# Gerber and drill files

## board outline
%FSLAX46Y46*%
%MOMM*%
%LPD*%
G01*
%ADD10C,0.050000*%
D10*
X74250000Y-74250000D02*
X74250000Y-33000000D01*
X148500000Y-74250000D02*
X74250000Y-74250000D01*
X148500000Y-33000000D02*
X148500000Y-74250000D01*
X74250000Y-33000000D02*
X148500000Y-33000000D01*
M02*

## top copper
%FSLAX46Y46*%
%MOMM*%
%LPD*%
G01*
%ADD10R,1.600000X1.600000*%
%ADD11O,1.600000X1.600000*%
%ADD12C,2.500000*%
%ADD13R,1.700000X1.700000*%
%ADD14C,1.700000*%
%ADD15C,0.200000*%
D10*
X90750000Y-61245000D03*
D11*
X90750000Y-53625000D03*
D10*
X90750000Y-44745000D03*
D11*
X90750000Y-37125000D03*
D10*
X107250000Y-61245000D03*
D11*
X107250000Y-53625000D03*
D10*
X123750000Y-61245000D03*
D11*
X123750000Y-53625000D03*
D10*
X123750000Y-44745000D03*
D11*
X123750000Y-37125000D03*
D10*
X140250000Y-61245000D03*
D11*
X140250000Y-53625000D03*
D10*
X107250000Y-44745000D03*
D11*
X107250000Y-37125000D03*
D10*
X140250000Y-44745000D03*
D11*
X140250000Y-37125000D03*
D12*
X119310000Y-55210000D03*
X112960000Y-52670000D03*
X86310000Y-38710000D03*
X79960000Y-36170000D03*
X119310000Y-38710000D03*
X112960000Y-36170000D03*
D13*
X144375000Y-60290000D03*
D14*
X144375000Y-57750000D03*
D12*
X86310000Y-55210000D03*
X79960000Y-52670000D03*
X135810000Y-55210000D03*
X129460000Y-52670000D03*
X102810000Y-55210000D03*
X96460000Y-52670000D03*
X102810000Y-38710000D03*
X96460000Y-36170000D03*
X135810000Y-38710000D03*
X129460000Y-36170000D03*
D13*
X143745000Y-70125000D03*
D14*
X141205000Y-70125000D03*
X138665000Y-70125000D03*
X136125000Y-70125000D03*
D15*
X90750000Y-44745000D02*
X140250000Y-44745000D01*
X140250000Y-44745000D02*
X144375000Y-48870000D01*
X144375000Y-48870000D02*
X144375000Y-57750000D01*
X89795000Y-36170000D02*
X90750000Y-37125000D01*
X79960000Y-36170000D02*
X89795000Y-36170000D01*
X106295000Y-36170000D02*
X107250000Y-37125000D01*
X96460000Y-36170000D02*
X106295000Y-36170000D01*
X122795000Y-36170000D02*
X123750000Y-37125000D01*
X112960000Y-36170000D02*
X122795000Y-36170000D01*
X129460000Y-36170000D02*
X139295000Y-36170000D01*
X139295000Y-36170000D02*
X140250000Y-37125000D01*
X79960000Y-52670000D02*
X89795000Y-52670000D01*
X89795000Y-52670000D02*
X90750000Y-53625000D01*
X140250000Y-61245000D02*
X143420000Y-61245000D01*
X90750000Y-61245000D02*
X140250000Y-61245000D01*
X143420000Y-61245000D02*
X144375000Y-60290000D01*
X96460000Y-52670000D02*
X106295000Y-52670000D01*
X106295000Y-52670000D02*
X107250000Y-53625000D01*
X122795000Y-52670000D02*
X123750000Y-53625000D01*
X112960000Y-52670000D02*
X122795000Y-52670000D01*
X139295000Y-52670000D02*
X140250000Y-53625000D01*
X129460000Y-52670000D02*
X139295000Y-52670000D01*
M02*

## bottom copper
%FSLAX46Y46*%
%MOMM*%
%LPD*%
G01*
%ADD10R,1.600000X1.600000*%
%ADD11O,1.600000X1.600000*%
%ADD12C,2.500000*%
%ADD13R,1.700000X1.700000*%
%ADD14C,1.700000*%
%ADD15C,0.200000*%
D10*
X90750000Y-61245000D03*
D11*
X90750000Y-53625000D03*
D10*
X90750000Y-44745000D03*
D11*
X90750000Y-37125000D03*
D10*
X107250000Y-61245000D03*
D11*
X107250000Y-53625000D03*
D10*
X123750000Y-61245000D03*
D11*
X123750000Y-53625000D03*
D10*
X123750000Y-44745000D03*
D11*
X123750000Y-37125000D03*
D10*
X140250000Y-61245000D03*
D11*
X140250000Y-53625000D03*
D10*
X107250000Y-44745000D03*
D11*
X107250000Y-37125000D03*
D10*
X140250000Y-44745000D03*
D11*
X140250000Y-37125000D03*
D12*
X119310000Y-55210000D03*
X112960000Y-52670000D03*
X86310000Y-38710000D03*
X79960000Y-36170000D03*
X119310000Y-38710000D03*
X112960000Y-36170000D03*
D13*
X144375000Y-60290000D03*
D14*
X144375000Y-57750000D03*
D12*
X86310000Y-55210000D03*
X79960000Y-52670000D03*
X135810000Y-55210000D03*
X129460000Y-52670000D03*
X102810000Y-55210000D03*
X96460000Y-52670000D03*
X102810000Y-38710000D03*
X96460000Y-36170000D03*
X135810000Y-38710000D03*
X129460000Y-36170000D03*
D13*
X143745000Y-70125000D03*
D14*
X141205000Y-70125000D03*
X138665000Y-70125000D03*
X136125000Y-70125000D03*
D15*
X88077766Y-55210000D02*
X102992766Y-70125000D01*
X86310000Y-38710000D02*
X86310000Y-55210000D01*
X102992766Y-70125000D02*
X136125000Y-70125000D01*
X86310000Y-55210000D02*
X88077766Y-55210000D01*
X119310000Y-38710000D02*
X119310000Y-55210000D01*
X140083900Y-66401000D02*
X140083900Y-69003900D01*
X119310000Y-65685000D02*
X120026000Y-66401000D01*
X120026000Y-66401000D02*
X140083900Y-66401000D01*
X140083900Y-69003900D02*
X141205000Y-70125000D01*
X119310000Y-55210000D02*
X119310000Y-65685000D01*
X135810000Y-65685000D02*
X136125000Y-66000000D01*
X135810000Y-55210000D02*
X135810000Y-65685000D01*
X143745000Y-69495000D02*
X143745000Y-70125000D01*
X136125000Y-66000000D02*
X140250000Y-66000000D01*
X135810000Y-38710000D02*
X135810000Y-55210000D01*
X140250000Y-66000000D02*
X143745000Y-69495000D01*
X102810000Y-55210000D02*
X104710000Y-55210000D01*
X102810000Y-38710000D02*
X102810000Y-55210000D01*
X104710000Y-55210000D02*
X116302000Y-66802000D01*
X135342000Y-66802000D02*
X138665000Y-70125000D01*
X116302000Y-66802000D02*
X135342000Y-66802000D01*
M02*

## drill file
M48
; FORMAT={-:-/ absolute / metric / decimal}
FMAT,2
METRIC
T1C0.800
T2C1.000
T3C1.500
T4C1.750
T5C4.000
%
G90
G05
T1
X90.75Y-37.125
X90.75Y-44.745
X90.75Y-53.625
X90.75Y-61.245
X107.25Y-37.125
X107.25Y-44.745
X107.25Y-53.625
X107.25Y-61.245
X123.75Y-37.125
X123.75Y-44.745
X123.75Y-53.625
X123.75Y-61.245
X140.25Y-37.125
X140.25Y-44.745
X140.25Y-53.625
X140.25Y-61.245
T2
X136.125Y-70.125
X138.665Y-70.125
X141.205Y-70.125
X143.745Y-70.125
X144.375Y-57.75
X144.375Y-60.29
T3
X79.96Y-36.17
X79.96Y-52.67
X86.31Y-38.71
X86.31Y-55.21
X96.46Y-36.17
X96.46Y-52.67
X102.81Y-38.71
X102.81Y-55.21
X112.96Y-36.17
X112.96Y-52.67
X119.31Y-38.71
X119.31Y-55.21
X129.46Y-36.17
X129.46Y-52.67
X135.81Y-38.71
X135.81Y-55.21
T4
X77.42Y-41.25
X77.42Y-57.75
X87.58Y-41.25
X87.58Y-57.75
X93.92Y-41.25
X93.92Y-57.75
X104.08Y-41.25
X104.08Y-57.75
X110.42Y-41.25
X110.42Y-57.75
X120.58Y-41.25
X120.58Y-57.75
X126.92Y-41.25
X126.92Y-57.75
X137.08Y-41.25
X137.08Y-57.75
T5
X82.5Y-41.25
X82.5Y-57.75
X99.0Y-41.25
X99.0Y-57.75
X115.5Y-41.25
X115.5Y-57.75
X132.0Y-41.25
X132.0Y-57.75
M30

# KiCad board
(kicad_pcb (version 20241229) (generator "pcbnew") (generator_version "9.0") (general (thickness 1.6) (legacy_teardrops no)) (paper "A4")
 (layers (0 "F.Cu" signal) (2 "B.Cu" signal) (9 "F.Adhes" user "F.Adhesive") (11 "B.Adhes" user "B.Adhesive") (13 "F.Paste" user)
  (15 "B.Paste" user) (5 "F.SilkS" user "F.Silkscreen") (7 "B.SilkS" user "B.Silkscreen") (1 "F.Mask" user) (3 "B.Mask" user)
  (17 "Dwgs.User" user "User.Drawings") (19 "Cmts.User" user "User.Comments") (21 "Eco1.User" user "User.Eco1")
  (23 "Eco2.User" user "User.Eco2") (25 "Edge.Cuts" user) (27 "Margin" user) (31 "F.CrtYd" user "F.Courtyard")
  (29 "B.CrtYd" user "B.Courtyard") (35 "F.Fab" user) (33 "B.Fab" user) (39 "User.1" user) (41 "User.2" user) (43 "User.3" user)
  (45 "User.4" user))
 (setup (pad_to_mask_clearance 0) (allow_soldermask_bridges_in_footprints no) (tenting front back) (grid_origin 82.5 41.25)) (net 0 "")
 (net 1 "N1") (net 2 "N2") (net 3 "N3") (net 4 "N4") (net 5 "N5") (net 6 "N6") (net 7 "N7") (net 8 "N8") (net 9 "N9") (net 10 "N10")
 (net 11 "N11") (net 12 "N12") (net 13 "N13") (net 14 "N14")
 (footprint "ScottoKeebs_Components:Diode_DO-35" (layer "F.Cu") (at 90.75 61.245 90)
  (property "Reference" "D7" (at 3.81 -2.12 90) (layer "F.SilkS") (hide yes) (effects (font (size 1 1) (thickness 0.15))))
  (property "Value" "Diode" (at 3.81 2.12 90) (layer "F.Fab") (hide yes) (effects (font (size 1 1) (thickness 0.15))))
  (pad "1" thru_hole rect (at 0 0 90) (size 1.6 1.6) (drill 0.8) (layers "*.Cu" "*.Mask") (remove_unused_layers no) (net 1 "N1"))
  (pad "2" thru_hole oval (at 7.62 0 90) (size 1.6 1.6) (drill 0.8) (layers "*.Cu" "*.Mask") (remove_unused_layers no) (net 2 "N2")))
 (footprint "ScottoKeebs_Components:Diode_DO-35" (layer "F.Cu") (at 90.75 44.745 90)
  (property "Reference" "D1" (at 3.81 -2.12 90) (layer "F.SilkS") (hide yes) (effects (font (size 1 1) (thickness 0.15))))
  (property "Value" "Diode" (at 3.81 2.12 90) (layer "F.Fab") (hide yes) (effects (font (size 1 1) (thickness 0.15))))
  (pad "1" thru_hole rect (at 0 0 90) (size 1.6 1.6) (drill 0.8) (layers "*.Cu" "*.Mask") (remove_unused_layers no) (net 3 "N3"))
  (pad "2" thru_hole oval (at 7.62 0 90) (size 1.6 1.6) (drill 0.8) (layers "*.Cu" "*.Mask") (remove_unused_layers no) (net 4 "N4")))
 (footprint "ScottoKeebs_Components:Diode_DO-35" (layer "F.Cu") (at 107.25 61.245 90)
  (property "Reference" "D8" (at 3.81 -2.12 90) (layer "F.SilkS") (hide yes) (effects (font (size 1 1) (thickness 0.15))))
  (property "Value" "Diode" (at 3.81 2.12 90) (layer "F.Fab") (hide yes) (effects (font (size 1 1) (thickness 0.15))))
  (pad "1" thru_hole rect (at 0 0 90) (size 1.6 1.6) (drill 0.8) (layers "*.Cu" "*.Mask") (remove_unused_layers no) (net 1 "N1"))
  (pad "2" thru_hole oval (at 7.62 0 90) (size 1.6 1.6) (drill 0.8) (layers "*.Cu" "*.Mask") (remove_unused_layers no) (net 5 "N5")))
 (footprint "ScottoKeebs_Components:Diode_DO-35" (layer "F.Cu") (at 123.75 61.245 90)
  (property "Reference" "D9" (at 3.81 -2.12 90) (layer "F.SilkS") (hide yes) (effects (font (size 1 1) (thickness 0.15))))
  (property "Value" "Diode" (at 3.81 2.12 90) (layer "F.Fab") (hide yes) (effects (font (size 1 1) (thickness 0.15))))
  (pad "1" thru_hole rect (at 0 0 90) (size 1.6 1.6) (drill 0.8) (layers "*.Cu" "*.Mask") (remove_unused_layers no) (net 1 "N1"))
  (pad "2" thru_hole oval (at 7.62 0 90) (size 1.6 1.6) (drill 0.8) (layers "*.Cu" "*.Mask") (remove_unused_layers no) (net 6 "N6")))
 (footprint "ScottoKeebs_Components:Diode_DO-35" (layer "F.Cu") (at 123.75 44.745 90)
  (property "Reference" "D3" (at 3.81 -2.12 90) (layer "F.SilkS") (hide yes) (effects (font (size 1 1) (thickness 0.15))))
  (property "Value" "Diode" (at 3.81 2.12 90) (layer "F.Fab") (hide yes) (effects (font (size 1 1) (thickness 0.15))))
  (pad "1" thru_hole rect (at 0 0 90) (size 1.6 1.6) (drill 0.8) (layers "*.Cu" "*.Mask") (remove_unused_layers no) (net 3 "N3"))
  (pad "2" thru_hole oval (at 7.62 0 90) (size 1.6 1.6) (drill 0.8) (layers "*.Cu" "*.Mask") (remove_unused_layers no) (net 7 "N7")))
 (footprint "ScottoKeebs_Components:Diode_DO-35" (layer "F.Cu") (at 140.25 61.245 90)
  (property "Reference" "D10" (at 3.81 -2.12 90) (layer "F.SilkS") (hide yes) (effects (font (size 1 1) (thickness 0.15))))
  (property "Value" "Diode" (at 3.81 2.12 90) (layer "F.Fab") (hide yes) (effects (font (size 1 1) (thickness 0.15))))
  (pad "1" thru_hole rect (at 0 0 90) (size 1.6 1.6) (drill 0.8) (layers "*.Cu" "*.Mask") (remove_unused_layers no) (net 1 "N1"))
  (pad "2" thru_hole oval (at 7.62 0 90) (size 1.6 1.6) (drill 0.8) (layers "*.Cu" "*.Mask") (remove_unused_layers no) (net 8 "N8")))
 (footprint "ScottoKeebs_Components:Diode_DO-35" (layer "F.Cu") (at 107.25 44.745 90)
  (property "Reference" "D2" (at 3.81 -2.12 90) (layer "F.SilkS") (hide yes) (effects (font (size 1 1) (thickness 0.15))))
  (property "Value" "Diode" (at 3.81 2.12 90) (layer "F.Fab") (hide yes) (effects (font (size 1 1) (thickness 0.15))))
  (pad "1" thru_hole rect (at 0 0 90) (size 1.6 1.6) (drill 0.8) (layers "*.Cu" "*.Mask") (remove_unused_layers no) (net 3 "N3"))
  (pad "2" thru_hole oval (at 7.62 0 90) (size 1.6 1.6) (drill 0.8) (layers "*.Cu" "*.Mask") (remove_unused_layers no) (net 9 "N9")))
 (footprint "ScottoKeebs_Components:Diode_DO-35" (layer "F.Cu") (at 140.25 44.745 90)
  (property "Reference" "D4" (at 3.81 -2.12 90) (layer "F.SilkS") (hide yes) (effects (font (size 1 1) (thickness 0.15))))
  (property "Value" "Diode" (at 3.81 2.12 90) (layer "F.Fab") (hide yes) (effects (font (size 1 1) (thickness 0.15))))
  (pad "1" thru_hole rect (at 0 0 90) (size 1.6 1.6) (drill 0.8) (layers "*.Cu" "*.Mask") (remove_unused_layers no) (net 3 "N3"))
  (pad "2" thru_hole oval (at 7.62 0 90) (size 1.6 1.6) (drill 0.8) (layers "*.Cu" "*.Mask") (remove_unused_layers no) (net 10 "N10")))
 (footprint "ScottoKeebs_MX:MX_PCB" (layer "B.Cu") (at 115.5 57.75 180)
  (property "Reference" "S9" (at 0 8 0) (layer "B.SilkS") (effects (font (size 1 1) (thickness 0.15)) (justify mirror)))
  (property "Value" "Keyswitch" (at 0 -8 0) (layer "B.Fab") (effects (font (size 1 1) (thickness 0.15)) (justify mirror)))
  (pad "" np_thru_hole circle (at -5.08 0 180) (size 1.75 1.75) (drill 1.75) (layers "*.Cu" "*.Mask"))
  (pad "" np_thru_hole circle (at 0 0 180) (size 4 4) (drill 4) (layers "*.Cu" "*.Mask"))
  (pad "" np_thru_hole circle (at 5.08 0 180) (size 1.75 1.75) (drill 1.75) (layers "*.Cu" "*.Mask"))
  (pad "1" thru_hole circle (at -3.81 2.54 180) (size 2.5 2.5) (drill 1.5) (layers "*.Cu" "*.Mask") (remove_unused_layers no) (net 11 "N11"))
  (pad "2" thru_hole circle (at 2.54 5.08 180) (size 2.5 2.5) (drill 1.5) (layers "*.Cu" "*.Mask") (remove_unused_layers no) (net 6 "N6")))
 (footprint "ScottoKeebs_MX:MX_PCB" (layer "B.Cu") (at 82.5 41.25 180)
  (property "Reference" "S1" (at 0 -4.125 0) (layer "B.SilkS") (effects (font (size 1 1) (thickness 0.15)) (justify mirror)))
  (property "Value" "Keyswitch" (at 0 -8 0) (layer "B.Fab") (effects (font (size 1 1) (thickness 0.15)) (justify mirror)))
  (pad "" np_thru_hole circle (at -5.08 0 180) (size 1.75 1.75) (drill 1.75) (layers "*.Cu" "*.Mask"))
  (pad "" np_thru_hole circle (at 0 0 180) (size 4 4) (drill 4) (layers "*.Cu" "*.Mask"))
  (pad "" np_thru_hole circle (at 5.08 0 180) (size 1.75 1.75) (drill 1.75) (layers "*.Cu" "*.Mask"))
  (pad "1" thru_hole circle (at -3.81 2.54 180) (size 2.5 2.5) (drill 1.5) (layers "*.Cu" "*.Mask") (remove_unused_layers no) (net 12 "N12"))
  (pad "2" thru_hole circle (at 2.54 5.08 180) (size 2.5 2.5) (drill 1.5) (layers "*.Cu" "*.Mask") (remove_unused_layers no) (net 4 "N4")))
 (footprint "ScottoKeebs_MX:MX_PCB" (layer "B.Cu") (at 115.5 41.25 180)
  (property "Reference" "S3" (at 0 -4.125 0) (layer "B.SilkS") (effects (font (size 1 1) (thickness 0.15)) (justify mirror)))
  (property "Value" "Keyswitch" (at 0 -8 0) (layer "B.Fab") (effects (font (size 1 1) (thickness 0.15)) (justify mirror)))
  (pad "" np_thru_hole circle (at -5.08 0 180) (size 1.75 1.75) (drill 1.75) (layers "*.Cu" "*.Mask"))
  (pad "" np_thru_hole circle (at 0 0 180) (size 4 4) (drill 4) (layers "*.Cu" "*.Mask"))
  (pad "" np_thru_hole circle (at 5.08 0 180) (size 1.75 1.75) (drill 1.75) (layers "*.Cu" "*.Mask"))
  (pad "1" thru_hole circle (at -3.81 2.54 180) (size 2.5 2.5) (drill 1.5) (layers "*.Cu" "*.Mask") (remove_unused_layers no) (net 11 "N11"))
  (pad "2" thru_hole circle (at 2.54 5.08 180) (size 2.5 2.5) (drill 1.5) (layers "*.Cu" "*.Mask") (remove_unused_layers no) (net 7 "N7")))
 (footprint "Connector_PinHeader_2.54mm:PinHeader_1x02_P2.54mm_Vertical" (layer "B.Cu") (at 144.375 60.29)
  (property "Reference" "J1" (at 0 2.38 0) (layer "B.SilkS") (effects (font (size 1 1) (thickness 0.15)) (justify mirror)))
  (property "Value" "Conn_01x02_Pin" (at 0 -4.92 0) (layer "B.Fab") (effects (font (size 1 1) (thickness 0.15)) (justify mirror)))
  (pad "1" thru_hole rect (at 0 0) (size 1.7 1.7) (drill 1) (layers "*.Cu" "*.Mask") (remove_unused_layers no) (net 1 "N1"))
  (pad "2" thru_hole circle (at 0 -2.54) (size 1.7 1.7) (drill 1) (layers "*.Cu" "*.Mask") (remove_unused_layers no) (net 3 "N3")))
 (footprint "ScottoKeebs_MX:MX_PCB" (layer "B.Cu") (at 82.5 57.75 180)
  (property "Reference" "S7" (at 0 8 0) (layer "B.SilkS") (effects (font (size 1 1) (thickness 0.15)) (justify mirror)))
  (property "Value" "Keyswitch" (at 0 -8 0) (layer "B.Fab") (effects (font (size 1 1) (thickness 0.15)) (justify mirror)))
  (pad "" np_thru_hole circle (at -5.08 0 180) (size 1.75 1.75) (drill 1.75) (layers "*.Cu" "*.Mask"))
  (pad "" np_thru_hole circle (at 0 0 180) (size 4 4) (drill 4) (layers "*.Cu" "*.Mask"))
  (pad "" np_thru_hole circle (at 5.08 0 180) (size 1.75 1.75) (drill 1.75) (layers "*.Cu" "*.Mask"))
  (pad "1" thru_hole circle (at -3.81 2.54 180) (size 2.5 2.5) (drill 1.5) (layers "*.Cu" "*.Mask") (remove_unused_layers no) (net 12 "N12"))
  (pad "2" thru_hole circle (at 2.54 5.08 180) (size 2.5 2.5) (drill 1.5) (layers "*.Cu" "*.Mask") (remove_unused_layers no) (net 2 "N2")))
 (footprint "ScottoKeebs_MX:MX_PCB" (layer "B.Cu") (at 132 57.75 180)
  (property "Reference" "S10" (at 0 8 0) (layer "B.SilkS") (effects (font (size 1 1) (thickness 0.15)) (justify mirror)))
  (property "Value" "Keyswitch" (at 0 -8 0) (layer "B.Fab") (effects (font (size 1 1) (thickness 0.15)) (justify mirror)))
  (pad "" np_thru_hole circle (at -5.08 0 180) (size 1.75 1.75) (drill 1.75) (layers "*.Cu" "*.Mask"))
  (pad "" np_thru_hole circle (at 0 0 180) (size 4 4) (drill 4) (layers "*.Cu" "*.Mask"))
  (pad "" np_thru_hole circle (at 5.08 0 180) (size 1.75 1.75) (drill 1.75) (layers "*.Cu" "*.Mask"))
  (pad "1" thru_hole circle (at -3.81 2.54 180) (size 2.5 2.5) (drill 1.5) (layers "*.Cu" "*.Mask") (remove_unused_layers no) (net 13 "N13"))
  (pad "2" thru_hole circle (at 2.54 5.08 180) (size 2.5 2.5) (drill 1.5) (layers "*.Cu" "*.Mask") (remove_unused_layers no) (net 8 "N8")))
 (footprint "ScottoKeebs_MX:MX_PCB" (layer "B.Cu") (at 99 57.75 180)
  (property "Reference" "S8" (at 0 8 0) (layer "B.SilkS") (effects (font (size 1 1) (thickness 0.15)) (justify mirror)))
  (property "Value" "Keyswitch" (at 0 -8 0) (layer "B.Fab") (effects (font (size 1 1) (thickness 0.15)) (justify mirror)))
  (pad "" np_thru_hole circle (at -5.08 0 180) (size 1.75 1.75) (drill 1.75) (layers "*.Cu" "*.Mask"))
  (pad "" np_thru_hole circle (at 0 0 180) (size 4 4) (drill 4) (layers "*.Cu" "*.Mask"))
  (pad "" np_thru_hole circle (at 5.08 0 180) (size 1.75 1.75) (drill 1.75) (layers "*.Cu" "*.Mask"))
  (pad "1" thru_hole circle (at -3.81 2.54 180) (size 2.5 2.5) (drill 1.5) (layers "*.Cu" "*.Mask") (remove_unused_layers no) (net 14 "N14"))
  (pad "2" thru_hole circle (at 2.54 5.08 180) (size 2.5 2.5) (drill 1.5) (layers "*.Cu" "*.Mask") (remove_unused_layers no) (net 5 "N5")))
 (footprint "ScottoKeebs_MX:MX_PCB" (layer "B.Cu") (at 99 41.25 180)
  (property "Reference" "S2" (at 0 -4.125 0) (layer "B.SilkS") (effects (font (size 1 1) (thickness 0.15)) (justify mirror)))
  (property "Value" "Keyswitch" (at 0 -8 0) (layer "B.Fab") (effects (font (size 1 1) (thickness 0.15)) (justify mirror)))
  (pad "" np_thru_hole circle (at -5.08 0 180) (size 1.75 1.75) (drill 1.75) (layers "*.Cu" "*.Mask"))
  (pad "" np_thru_hole circle (at 0 0 180) (size 4 4) (drill 4) (layers "*.Cu" "*.Mask"))
  (pad "" np_thru_hole circle (at 5.08 0 180) (size 1.75 1.75) (drill 1.75) (layers "*.Cu" "*.Mask"))
  (pad "1" thru_hole circle (at -3.81 2.54 180) (size 2.5 2.5) (drill 1.5) (layers "*.Cu" "*.Mask") (remove_unused_layers no) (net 14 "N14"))
  (pad "2" thru_hole circle (at 2.54 5.08 180) (size 2.5 2.5) (drill 1.5) (layers "*.Cu" "*.Mask") (remove_unused_layers no) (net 9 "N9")))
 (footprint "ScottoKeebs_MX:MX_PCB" (layer "B.Cu") (at 132 41.25 180)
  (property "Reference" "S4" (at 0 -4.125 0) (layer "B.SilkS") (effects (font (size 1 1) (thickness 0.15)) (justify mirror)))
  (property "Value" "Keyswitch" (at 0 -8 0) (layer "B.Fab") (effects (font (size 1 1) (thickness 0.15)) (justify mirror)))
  (pad "" np_thru_hole circle (at -5.08 0 180) (size 1.75 1.75) (drill 1.75) (layers "*.Cu" "*.Mask"))
  (pad "" np_thru_hole circle (at 0 0 180) (size 4 4) (drill 4) (layers "*.Cu" "*.Mask"))
  (pad "" np_thru_hole circle (at 5.08 0 180) (size 1.75 1.75) (drill 1.75) (layers "*.Cu" "*.Mask"))
  (pad "1" thru_hole circle (at -3.81 2.54 180) (size 2.5 2.5) (drill 1.5) (layers "*.Cu" "*.Mask") (remove_unused_layers no) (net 13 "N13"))
  (pad "2" thru_hole circle (at 2.54 5.08 180) (size 2.5 2.5) (drill 1.5) (layers "*.Cu" "*.Mask") (remove_unused_layers no) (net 10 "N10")))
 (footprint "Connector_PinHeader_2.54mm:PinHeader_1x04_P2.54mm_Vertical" (layer "B.Cu") (at 143.745 70.125 90)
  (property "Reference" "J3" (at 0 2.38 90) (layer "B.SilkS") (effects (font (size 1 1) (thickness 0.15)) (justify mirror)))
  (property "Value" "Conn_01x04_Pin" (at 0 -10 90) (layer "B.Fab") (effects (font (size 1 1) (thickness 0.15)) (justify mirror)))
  (pad "1" thru_hole rect (at 0 0 90) (size 1.7 1.7) (drill 1) (layers "*.Cu" "*.Mask") (remove_unused_layers no) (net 13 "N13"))
  (pad "2" thru_hole circle (at 0 -2.54 90) (size 1.7 1.7) (drill 1) (layers "*.Cu" "*.Mask") (remove_unused_layers no) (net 11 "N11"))
  (pad "3" thru_hole circle (at 0 -5.08 90) (size 1.7 1.7) (drill 1) (layers "*.Cu" "*.Mask") (remove_unused_layers no) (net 14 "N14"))
  (pad "4" thru_hole circle (at 0 -7.62 90) (size 1.7 1.7) (drill 1) (layers "*.Cu" "*.Mask") (remove_unused_layers no) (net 12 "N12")))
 (gr_line (start 74.25 74.25) (end 74.25 33) (stroke (width 0.05) (type default)) (layer "Edge.Cuts"))
 (gr_line (start 148.5 74.25) (end 74.25 74.25) (stroke (width 0.05) (type default)) (layer "Edge.Cuts"))
 (gr_line (start 148.5 33) (end 148.5 74.25) (stroke (width 0.05) (type default)) (layer "Edge.Cuts"))
 (gr_line (start 74.25 33) (end 148.5 33) (stroke (width 0.05) (type default)) (layer "Edge.Cuts"))
 (segment (start 90.75 44.745) (end 140.25 44.745) (width 0.2) (layer "F.Cu") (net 3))
 (segment (start 140.25 44.745) (end 144.375 48.87) (width 0.2) (layer "F.Cu") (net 3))
 (segment (start 144.375 48.87) (end 144.375 57.75) (width 0.2) (layer "F.Cu") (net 3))
 (segment (start 89.795 36.17) (end 90.75 37.125) (width 0.2) (layer "F.Cu") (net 4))
 (segment (start 79.96 36.17) (end 89.795 36.17) (width 0.2) (layer "F.Cu") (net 4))
 (segment (start 106.295 36.17) (end 107.25 37.125) (width 0.2) (layer "F.Cu") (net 9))
 (segment (start 96.46 36.17) (end 106.295 36.17) (width 0.2) (layer "F.Cu") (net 9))
 (segment (start 122.795 36.17) (end 123.75 37.125) (width 0.2) (layer "F.Cu") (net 7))
 (segment (start 112.96 36.17) (end 122.795 36.17) (width 0.2) (layer "F.Cu") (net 7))
 (segment (start 129.46 36.17) (end 139.295 36.17) (width 0.2) (layer "F.Cu") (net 10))
 (segment (start 139.295 36.17) (end 140.25 37.125) (width 0.2) (layer "F.Cu") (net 10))
 (segment (start 79.96 52.67) (end 89.795 52.67) (width 0.2) (layer "F.Cu") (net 2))
 (segment (start 89.795 52.67) (end 90.75 53.625) (width 0.2) (layer "F.Cu") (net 2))
 (segment (start 140.25 61.245) (end 143.42 61.245) (width 0.2) (layer "F.Cu") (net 1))
 (segment (start 90.75 61.245) (end 140.25 61.245) (width 0.2) (layer "F.Cu") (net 1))
 (segment (start 143.42 61.245) (end 144.375 60.29) (width 0.2) (layer "F.Cu") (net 1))
 (segment (start 96.46 52.67) (end 106.295 52.67) (width 0.2) (layer "F.Cu") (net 5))
 (segment (start 106.295 52.67) (end 107.25 53.625) (width 0.2) (layer "F.Cu") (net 5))
 (segment (start 122.795 52.67) (end 123.75 53.625) (width 0.2) (layer "F.Cu") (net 6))
 (segment (start 112.96 52.67) (end 122.795 52.67) (width 0.2) (layer "F.Cu") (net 6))
 (segment (start 139.295 52.67) (end 140.25 53.625) (width 0.2) (layer "F.Cu") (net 8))
 (segment (start 129.46 52.67) (end 139.295 52.67) (width 0.2) (layer "F.Cu") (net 8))
 (segment (start 88.077766 55.21) (end 102.992766 70.125) (width 0.2) (layer "B.Cu") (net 12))
 (segment (start 86.31 38.71) (end 86.31 55.21) (width 0.2) (layer "B.Cu") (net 12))
 (segment (start 102.992766 70.125) (end 136.125 70.125) (width 0.2) (layer "B.Cu") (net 12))
 (segment (start 86.31 55.21) (end 88.077766 55.21) (width 0.2) (layer "B.Cu") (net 12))
 (segment (start 119.31 38.71) (end 119.31 55.21) (width 0.2) (layer "B.Cu") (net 11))
 (segment (start 140.0839 66.401) (end 140.0839 69.0039) (width 0.2) (layer "B.Cu") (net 11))
 (segment (start 119.31 65.685) (end 120.026 66.401) (width 0.2) (layer "B.Cu") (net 11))
 (segment (start 120.026 66.401) (end 140.0839 66.401) (width 0.2) (layer "B.Cu") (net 11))
 (segment (start 140.0839 69.0039) (end 141.205 70.125) (width 0.2) (layer "B.Cu") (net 11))
 (segment (start 119.31 55.21) (end 119.31 65.685) (width 0.2) (layer "B.Cu") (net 11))
 (segment (start 135.81 65.685) (end 136.125 66) (width 0.2) (layer "B.Cu") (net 13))
 (segment (start 135.81 55.21) (end 135.81 65.685) (width 0.2) (layer "B.Cu") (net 13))
 (segment (start 143.745 69.495) (end 143.745 70.125) (width 0.2) (layer "B.Cu") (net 13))
 (segment (start 136.125 66) (end 140.25 66) (width 0.2) (layer "B.Cu") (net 13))
 (segment (start 135.81 38.71) (end 135.81 55.21) (width 0.2) (layer "B.Cu") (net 13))
 (segment (start 140.25 66) (end 143.745 69.495) (width 0.2) (layer "B.Cu") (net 13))
 (segment (start 102.81 55.21) (end 104.71 55.21) (width 0.2) (layer "B.Cu") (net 14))
 (segment (start 102.81 38.71) (end 102.81 55.21) (width 0.2) (layer "B.Cu") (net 14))
 (segment (start 104.71 55.21) (end 116.302 66.802) (width 0.2) (layer "B.Cu") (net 14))
 (segment (start 135.342 66.802) (end 138.665 70.125) (width 0.2) (layer "B.Cu") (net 14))
 (segment (start 116.302 66.802) (end 135.342 66.802) (width 0.2) (layer "B.Cu") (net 14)))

